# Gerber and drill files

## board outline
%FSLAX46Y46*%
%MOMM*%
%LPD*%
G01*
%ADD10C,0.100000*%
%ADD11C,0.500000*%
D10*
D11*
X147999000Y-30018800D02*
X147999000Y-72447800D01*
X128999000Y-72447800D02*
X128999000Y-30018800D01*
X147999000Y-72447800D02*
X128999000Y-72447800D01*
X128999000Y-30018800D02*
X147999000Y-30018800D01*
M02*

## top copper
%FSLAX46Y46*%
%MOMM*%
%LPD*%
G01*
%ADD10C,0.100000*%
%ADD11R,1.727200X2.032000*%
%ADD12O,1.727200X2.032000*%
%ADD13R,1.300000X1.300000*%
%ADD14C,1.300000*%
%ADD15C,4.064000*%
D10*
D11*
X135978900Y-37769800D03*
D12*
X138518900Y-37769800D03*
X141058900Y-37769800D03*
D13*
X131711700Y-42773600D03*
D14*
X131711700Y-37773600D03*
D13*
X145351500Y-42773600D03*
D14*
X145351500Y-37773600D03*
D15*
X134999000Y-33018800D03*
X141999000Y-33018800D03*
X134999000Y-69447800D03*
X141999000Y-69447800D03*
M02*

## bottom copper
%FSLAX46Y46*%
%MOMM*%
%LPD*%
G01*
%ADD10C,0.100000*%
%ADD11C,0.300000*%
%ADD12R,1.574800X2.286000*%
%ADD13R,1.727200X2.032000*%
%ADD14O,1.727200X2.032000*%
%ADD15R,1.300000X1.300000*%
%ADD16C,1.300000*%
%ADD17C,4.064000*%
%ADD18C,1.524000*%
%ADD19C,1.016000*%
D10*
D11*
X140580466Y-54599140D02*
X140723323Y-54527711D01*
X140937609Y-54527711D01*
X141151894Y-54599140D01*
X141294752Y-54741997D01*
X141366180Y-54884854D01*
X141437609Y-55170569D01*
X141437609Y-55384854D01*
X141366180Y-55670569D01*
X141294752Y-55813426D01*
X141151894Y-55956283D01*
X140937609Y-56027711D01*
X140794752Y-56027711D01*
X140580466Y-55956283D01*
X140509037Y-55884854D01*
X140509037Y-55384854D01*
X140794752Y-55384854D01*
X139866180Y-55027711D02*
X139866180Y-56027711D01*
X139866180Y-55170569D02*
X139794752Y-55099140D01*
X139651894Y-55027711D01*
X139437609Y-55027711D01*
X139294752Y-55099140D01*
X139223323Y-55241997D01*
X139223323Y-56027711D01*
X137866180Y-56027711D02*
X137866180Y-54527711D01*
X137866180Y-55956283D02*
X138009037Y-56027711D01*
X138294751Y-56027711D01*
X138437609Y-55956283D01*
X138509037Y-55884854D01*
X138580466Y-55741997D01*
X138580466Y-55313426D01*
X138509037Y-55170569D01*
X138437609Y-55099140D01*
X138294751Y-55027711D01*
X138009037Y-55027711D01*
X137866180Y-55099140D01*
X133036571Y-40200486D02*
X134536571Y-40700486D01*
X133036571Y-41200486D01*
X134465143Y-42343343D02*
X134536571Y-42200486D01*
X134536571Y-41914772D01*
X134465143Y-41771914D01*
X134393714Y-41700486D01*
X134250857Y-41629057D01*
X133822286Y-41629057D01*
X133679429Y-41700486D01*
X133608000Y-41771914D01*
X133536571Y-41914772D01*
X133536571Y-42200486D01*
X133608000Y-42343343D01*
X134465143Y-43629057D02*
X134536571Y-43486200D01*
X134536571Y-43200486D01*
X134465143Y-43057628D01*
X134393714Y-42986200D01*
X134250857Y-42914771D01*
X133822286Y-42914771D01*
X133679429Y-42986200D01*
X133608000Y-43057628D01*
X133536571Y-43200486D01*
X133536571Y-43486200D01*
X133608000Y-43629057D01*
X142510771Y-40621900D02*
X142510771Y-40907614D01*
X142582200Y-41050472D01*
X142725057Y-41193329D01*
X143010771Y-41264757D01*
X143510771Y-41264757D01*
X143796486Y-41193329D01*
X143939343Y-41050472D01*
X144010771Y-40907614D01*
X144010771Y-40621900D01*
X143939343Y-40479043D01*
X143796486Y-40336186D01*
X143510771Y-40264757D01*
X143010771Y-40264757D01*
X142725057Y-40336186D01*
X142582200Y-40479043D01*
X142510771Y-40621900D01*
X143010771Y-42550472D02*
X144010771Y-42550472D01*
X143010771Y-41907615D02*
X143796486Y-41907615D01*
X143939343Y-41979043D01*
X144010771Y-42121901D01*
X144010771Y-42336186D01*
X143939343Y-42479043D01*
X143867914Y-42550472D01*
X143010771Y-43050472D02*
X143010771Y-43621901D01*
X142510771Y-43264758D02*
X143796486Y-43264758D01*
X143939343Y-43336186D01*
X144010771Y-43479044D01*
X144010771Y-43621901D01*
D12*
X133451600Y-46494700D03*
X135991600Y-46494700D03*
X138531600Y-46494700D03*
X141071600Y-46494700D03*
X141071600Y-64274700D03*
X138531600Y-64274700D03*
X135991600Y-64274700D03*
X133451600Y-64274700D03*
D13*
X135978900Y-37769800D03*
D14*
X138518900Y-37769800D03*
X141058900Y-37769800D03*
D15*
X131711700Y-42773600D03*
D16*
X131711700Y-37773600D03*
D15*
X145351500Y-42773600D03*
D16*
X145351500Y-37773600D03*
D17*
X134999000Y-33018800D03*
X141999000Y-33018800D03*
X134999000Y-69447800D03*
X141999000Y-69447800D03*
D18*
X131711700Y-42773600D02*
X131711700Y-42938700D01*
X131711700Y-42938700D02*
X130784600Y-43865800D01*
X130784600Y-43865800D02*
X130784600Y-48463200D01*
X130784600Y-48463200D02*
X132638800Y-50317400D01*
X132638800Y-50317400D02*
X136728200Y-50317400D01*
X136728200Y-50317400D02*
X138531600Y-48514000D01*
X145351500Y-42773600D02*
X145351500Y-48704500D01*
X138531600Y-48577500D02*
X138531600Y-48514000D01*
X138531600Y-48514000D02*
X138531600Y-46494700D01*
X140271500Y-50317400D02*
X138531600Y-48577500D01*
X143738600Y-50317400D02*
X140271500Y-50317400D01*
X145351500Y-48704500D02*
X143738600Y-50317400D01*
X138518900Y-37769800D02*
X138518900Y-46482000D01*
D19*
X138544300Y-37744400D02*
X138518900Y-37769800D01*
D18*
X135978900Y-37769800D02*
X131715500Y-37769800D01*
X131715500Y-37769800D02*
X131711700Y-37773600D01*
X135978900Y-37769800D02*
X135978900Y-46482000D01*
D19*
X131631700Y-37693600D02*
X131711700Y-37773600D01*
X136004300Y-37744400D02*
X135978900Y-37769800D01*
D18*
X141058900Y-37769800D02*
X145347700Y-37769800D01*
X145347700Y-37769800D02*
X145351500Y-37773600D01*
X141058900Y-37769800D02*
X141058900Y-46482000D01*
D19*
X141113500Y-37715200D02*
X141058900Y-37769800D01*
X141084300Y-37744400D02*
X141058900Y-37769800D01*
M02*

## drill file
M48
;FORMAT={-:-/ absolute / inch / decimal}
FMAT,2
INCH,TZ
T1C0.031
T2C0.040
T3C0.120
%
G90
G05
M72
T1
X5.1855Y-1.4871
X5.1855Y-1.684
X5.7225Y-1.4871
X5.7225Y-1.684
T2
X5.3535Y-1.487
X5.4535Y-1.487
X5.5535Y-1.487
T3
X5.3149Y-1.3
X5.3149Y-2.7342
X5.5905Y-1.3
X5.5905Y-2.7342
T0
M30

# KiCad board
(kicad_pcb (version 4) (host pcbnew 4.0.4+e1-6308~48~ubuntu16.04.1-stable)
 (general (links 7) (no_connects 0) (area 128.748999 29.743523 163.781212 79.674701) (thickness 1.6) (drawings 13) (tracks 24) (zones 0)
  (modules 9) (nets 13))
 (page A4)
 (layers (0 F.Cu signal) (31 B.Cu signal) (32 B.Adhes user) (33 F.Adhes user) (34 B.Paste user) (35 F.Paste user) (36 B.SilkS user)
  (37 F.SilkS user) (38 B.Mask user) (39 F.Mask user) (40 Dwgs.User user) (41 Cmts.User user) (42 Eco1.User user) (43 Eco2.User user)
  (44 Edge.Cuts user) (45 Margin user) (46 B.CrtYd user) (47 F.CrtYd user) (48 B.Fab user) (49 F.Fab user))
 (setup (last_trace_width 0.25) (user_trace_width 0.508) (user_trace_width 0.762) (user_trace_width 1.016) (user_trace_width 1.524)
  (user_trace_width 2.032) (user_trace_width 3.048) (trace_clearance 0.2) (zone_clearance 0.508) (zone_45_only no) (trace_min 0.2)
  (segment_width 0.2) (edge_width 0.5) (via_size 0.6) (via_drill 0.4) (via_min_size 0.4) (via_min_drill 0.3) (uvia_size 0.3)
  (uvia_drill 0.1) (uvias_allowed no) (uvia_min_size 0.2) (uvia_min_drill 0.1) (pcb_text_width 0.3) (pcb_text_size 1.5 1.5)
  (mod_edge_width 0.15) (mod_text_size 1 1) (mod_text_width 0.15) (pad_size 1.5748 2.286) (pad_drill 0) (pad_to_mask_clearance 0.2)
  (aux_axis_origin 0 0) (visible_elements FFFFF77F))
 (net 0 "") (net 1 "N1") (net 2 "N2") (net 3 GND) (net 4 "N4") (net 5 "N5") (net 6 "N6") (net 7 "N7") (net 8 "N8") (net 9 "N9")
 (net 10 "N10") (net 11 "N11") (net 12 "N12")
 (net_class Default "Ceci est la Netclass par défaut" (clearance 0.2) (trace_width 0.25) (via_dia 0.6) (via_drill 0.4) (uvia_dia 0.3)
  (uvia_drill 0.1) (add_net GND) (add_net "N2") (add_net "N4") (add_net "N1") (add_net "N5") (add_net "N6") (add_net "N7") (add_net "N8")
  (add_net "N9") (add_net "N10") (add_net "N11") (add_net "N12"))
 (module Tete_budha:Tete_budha (layer F.Cu) (at 142.3543 55.26532 270)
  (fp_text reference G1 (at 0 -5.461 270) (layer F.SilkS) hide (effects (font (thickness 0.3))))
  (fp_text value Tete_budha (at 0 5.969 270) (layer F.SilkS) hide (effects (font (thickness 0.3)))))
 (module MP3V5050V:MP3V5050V (layer B.Cu) (at 137.2616 55.3847)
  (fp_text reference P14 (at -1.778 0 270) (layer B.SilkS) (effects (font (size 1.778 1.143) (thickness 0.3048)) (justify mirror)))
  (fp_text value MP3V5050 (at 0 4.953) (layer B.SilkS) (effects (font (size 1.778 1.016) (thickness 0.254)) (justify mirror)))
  (pad 1 smd rect (at -3.81 -8.89) (size 1.5748 2.286) (layers B.Cu B.Paste B.Mask) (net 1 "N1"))
  (pad 2 smd rect (at -1.27 -8.89) (size 1.5748 2.286) (layers B.Cu B.Paste B.Mask) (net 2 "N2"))
  (pad 3 smd rect (at 1.27 -8.89) (size 1.5748 2.286) (layers B.Cu B.Paste B.Mask) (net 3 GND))
  (pad 4 smd rect (at 3.81 -8.89) (size 1.5748 2.286) (layers B.Cu B.Paste B.Mask) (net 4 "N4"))
  (pad 5 smd rect (at 3.81 8.89) (size 1.5748 2.286) (layers B.Cu B.Paste B.Mask) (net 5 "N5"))
  (pad 6 smd rect (at 1.27 8.89) (size 1.5748 2.286) (layers B.Cu B.Paste B.Mask) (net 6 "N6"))
  (pad 7 smd rect (at -1.27 8.89) (size 1.5748 2.286) (layers B.Cu B.Paste B.Mask) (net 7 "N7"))
  (pad 8 smd rect (at -3.81 8.89) (size 1.5748 2.286) (layers B.Cu B.Paste B.Mask) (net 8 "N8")))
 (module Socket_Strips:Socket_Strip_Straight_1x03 (layer F.Cu) (at 135.9789 37.7698)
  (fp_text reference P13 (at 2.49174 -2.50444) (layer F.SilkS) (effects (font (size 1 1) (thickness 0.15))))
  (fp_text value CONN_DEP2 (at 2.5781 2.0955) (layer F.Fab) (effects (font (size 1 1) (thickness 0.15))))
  (pad 1 thru_hole rect (at 0 0) (size 1.7272 2.032) (drill 1.016) (layers *.Cu *.Mask F.SilkS) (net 2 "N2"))
  (pad 2 thru_hole oval (at 2.54 0) (size 1.7272 2.032) (drill 1.016) (layers *.Cu *.Mask F.SilkS) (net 3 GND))
  (pad 3 thru_hole oval (at 5.08 0) (size 1.7272 2.032) (drill 1.016) (layers *.Cu *.Mask F.SilkS) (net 4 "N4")))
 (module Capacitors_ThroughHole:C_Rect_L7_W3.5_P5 (layer F.Cu) (at 131.7117 42.7736 90)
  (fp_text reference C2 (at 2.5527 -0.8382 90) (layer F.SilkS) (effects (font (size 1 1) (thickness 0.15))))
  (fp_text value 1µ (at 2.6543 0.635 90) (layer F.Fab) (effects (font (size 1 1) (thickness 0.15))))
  (pad 1 thru_hole rect (at 0 0 90) (size 1.3 1.3) (drill 0.8) (layers *.Cu *.Mask F.SilkS) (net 3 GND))
  (pad 2 thru_hole circle (at 5 0 90) (size 1.3 1.3) (drill 0.8) (layers *.Cu *.Mask F.SilkS) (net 2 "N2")))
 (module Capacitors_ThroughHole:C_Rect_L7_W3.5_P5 (layer F.Cu) (at 145.3515 42.7736 90)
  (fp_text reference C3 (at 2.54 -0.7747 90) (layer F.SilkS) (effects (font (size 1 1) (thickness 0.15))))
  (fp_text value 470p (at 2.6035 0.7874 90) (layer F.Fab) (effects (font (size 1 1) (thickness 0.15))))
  (pad 1 thru_hole rect (at 0 0 90) (size 1.3 1.3) (drill 0.8) (layers *.Cu *.Mask F.SilkS) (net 3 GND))
  (pad 2 thru_hole circle (at 5 0 90) (size 1.3 1.3) (drill 0.8) (layers *.Cu *.Mask F.SilkS) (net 4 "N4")))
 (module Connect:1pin (layer F.Cu) (at 134.999 33.0188)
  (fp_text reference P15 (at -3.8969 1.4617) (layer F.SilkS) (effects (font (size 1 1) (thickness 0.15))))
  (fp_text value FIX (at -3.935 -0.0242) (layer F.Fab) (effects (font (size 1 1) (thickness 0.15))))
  (pad 1 thru_hole circle (at 0 0) (size 4.064 4.064) (drill 3.048) (layers *.Cu *.Mask F.SilkS) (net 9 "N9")))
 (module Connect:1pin (layer F.Cu) (at 141.999 33.0188)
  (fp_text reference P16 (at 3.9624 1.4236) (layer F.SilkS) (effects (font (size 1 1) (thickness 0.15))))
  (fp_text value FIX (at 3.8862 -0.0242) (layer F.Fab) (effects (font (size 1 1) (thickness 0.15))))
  (pad 1 thru_hole circle (at 0 0) (size 4.064 4.064) (drill 3.048) (layers *.Cu *.Mask F.SilkS) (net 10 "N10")))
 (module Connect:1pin (layer F.Cu) (at 134.999 69.4478)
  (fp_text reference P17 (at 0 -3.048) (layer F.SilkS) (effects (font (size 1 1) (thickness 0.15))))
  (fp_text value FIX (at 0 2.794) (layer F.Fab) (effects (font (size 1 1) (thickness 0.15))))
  (pad 1 thru_hole circle (at 0 0) (size 4.064 4.064) (drill 3.048) (layers *.Cu *.Mask F.SilkS) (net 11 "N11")))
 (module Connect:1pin (layer F.Cu) (at 141.999 69.4478)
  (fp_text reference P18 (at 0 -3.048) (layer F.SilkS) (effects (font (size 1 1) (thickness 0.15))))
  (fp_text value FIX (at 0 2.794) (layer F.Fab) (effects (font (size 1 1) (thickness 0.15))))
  (pad 1 thru_hole circle (at 0 0) (size 4.064 4.064) (drill 3.048) (layers *.Cu *.Mask F.SilkS) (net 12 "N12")))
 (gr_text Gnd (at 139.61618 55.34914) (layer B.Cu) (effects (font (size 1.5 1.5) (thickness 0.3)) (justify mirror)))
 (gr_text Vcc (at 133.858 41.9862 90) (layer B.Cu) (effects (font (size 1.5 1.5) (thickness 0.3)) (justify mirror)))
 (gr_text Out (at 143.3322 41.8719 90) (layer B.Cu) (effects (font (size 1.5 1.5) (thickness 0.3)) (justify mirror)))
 (gr_line (start 147.999 30.0188) (end 147.999 72.4478) (angle 90) (layer Edge.Cuts) (width 0.5))
 (gr_line (start 128.999 72.4478) (end 128.999 30.0188) (angle 90) (layer Edge.Cuts) (width 0.5))
 (gr_line (start 147.999 72.4478) (end 128.999 72.4478) (angle 90) (layer Edge.Cuts) (width 0.5))
 (gr_line (start 128.999 30.0188) (end 147.999 30.0188) (angle 90) (layer Edge.Cuts) (width 0.5))
 (segment (start 131.7117 42.7736) (end 131.7117 42.9387) (width 1.524) (layer B.Cu) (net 3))
 (segment (start 131.7117 42.9387) (end 130.7846 43.8658) (width 1.524) (layer B.Cu) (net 3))
 (segment (start 130.7846 43.8658) (end 130.7846 48.4632) (width 1.524) (layer B.Cu) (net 3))
 (segment (start 130.7846 48.4632) (end 132.6388 50.3174) (width 1.524) (layer B.Cu) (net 3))
 (segment (start 132.6388 50.3174) (end 136.7282 50.3174) (width 1.524) (layer B.Cu) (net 3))
 (segment (start 136.7282 50.3174) (end 138.5316 48.514) (width 1.524) (layer B.Cu) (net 3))
 (segment (start 145.3515 42.7736) (end 145.3515 48.7045) (width 1.524) (layer B.Cu) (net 3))
 (segment (start 138.5316 48.5775) (end 138.5316 48.514) (width 1.524) (layer B.Cu) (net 3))
 (segment (start 138.5316 48.514) (end 138.5316 46.4947) (width 1.524) (layer B.Cu) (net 3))
 (segment (start 140.2715 50.3174) (end 138.5316 48.5775) (width 1.524) (layer B.Cu) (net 3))
 (segment (start 143.7386 50.3174) (end 140.2715 50.3174) (width 1.524) (layer B.Cu) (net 3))
 (segment (start 145.3515 48.7045) (end 143.7386 50.3174) (width 1.524) (layer B.Cu) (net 3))
 (segment (start 138.5189 37.7698) (end 138.5189 46.482) (width 1.524) (layer B.Cu) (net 3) (status 10))
 (segment (start 138.5443 37.7444) (end 138.5189 37.7698) (width 1.016) (layer B.Cu) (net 3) (status 30))
 (segment (start 135.9789 37.7698) (end 131.7155 37.7698) (width 1.524) (layer B.Cu) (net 2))
 (segment (start 131.7155 37.7698) (end 131.7117 37.7736) (width 1.524) (layer B.Cu) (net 2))
 (segment (start 135.9789 37.7698) (end 135.9789 46.482) (width 1.524) (layer B.Cu) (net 2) (status 10))
 (segment (start 131.6317 37.6936) (end 131.7117 37.7736) (width 1.016) (layer B.Cu) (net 2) (status 30))
 (segment (start 136.0043 37.7444) (end 135.9789 37.7698) (width 1.016) (layer B.Cu) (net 2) (status 30))
 (segment (start 141.0589 37.7698) (end 145.3477 37.7698) (width 1.524) (layer B.Cu) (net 4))
 (segment (start 145.3477 37.7698) (end 145.3515 37.7736) (width 1.524) (layer B.Cu) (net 4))
 (segment (start 141.0589 37.7698) (end 141.0589 46.482) (width 1.524) (layer B.Cu) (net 4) (status 10))
 (segment (start 141.1135 37.7152) (end 141.0589 37.7698) (width 1.016) (layer B.Cu) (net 4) (status 30))
 (segment (start 141.0843 37.7444) (end 141.0589 37.7698) (width 1.016) (layer B.Cu) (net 4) (status 30)))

